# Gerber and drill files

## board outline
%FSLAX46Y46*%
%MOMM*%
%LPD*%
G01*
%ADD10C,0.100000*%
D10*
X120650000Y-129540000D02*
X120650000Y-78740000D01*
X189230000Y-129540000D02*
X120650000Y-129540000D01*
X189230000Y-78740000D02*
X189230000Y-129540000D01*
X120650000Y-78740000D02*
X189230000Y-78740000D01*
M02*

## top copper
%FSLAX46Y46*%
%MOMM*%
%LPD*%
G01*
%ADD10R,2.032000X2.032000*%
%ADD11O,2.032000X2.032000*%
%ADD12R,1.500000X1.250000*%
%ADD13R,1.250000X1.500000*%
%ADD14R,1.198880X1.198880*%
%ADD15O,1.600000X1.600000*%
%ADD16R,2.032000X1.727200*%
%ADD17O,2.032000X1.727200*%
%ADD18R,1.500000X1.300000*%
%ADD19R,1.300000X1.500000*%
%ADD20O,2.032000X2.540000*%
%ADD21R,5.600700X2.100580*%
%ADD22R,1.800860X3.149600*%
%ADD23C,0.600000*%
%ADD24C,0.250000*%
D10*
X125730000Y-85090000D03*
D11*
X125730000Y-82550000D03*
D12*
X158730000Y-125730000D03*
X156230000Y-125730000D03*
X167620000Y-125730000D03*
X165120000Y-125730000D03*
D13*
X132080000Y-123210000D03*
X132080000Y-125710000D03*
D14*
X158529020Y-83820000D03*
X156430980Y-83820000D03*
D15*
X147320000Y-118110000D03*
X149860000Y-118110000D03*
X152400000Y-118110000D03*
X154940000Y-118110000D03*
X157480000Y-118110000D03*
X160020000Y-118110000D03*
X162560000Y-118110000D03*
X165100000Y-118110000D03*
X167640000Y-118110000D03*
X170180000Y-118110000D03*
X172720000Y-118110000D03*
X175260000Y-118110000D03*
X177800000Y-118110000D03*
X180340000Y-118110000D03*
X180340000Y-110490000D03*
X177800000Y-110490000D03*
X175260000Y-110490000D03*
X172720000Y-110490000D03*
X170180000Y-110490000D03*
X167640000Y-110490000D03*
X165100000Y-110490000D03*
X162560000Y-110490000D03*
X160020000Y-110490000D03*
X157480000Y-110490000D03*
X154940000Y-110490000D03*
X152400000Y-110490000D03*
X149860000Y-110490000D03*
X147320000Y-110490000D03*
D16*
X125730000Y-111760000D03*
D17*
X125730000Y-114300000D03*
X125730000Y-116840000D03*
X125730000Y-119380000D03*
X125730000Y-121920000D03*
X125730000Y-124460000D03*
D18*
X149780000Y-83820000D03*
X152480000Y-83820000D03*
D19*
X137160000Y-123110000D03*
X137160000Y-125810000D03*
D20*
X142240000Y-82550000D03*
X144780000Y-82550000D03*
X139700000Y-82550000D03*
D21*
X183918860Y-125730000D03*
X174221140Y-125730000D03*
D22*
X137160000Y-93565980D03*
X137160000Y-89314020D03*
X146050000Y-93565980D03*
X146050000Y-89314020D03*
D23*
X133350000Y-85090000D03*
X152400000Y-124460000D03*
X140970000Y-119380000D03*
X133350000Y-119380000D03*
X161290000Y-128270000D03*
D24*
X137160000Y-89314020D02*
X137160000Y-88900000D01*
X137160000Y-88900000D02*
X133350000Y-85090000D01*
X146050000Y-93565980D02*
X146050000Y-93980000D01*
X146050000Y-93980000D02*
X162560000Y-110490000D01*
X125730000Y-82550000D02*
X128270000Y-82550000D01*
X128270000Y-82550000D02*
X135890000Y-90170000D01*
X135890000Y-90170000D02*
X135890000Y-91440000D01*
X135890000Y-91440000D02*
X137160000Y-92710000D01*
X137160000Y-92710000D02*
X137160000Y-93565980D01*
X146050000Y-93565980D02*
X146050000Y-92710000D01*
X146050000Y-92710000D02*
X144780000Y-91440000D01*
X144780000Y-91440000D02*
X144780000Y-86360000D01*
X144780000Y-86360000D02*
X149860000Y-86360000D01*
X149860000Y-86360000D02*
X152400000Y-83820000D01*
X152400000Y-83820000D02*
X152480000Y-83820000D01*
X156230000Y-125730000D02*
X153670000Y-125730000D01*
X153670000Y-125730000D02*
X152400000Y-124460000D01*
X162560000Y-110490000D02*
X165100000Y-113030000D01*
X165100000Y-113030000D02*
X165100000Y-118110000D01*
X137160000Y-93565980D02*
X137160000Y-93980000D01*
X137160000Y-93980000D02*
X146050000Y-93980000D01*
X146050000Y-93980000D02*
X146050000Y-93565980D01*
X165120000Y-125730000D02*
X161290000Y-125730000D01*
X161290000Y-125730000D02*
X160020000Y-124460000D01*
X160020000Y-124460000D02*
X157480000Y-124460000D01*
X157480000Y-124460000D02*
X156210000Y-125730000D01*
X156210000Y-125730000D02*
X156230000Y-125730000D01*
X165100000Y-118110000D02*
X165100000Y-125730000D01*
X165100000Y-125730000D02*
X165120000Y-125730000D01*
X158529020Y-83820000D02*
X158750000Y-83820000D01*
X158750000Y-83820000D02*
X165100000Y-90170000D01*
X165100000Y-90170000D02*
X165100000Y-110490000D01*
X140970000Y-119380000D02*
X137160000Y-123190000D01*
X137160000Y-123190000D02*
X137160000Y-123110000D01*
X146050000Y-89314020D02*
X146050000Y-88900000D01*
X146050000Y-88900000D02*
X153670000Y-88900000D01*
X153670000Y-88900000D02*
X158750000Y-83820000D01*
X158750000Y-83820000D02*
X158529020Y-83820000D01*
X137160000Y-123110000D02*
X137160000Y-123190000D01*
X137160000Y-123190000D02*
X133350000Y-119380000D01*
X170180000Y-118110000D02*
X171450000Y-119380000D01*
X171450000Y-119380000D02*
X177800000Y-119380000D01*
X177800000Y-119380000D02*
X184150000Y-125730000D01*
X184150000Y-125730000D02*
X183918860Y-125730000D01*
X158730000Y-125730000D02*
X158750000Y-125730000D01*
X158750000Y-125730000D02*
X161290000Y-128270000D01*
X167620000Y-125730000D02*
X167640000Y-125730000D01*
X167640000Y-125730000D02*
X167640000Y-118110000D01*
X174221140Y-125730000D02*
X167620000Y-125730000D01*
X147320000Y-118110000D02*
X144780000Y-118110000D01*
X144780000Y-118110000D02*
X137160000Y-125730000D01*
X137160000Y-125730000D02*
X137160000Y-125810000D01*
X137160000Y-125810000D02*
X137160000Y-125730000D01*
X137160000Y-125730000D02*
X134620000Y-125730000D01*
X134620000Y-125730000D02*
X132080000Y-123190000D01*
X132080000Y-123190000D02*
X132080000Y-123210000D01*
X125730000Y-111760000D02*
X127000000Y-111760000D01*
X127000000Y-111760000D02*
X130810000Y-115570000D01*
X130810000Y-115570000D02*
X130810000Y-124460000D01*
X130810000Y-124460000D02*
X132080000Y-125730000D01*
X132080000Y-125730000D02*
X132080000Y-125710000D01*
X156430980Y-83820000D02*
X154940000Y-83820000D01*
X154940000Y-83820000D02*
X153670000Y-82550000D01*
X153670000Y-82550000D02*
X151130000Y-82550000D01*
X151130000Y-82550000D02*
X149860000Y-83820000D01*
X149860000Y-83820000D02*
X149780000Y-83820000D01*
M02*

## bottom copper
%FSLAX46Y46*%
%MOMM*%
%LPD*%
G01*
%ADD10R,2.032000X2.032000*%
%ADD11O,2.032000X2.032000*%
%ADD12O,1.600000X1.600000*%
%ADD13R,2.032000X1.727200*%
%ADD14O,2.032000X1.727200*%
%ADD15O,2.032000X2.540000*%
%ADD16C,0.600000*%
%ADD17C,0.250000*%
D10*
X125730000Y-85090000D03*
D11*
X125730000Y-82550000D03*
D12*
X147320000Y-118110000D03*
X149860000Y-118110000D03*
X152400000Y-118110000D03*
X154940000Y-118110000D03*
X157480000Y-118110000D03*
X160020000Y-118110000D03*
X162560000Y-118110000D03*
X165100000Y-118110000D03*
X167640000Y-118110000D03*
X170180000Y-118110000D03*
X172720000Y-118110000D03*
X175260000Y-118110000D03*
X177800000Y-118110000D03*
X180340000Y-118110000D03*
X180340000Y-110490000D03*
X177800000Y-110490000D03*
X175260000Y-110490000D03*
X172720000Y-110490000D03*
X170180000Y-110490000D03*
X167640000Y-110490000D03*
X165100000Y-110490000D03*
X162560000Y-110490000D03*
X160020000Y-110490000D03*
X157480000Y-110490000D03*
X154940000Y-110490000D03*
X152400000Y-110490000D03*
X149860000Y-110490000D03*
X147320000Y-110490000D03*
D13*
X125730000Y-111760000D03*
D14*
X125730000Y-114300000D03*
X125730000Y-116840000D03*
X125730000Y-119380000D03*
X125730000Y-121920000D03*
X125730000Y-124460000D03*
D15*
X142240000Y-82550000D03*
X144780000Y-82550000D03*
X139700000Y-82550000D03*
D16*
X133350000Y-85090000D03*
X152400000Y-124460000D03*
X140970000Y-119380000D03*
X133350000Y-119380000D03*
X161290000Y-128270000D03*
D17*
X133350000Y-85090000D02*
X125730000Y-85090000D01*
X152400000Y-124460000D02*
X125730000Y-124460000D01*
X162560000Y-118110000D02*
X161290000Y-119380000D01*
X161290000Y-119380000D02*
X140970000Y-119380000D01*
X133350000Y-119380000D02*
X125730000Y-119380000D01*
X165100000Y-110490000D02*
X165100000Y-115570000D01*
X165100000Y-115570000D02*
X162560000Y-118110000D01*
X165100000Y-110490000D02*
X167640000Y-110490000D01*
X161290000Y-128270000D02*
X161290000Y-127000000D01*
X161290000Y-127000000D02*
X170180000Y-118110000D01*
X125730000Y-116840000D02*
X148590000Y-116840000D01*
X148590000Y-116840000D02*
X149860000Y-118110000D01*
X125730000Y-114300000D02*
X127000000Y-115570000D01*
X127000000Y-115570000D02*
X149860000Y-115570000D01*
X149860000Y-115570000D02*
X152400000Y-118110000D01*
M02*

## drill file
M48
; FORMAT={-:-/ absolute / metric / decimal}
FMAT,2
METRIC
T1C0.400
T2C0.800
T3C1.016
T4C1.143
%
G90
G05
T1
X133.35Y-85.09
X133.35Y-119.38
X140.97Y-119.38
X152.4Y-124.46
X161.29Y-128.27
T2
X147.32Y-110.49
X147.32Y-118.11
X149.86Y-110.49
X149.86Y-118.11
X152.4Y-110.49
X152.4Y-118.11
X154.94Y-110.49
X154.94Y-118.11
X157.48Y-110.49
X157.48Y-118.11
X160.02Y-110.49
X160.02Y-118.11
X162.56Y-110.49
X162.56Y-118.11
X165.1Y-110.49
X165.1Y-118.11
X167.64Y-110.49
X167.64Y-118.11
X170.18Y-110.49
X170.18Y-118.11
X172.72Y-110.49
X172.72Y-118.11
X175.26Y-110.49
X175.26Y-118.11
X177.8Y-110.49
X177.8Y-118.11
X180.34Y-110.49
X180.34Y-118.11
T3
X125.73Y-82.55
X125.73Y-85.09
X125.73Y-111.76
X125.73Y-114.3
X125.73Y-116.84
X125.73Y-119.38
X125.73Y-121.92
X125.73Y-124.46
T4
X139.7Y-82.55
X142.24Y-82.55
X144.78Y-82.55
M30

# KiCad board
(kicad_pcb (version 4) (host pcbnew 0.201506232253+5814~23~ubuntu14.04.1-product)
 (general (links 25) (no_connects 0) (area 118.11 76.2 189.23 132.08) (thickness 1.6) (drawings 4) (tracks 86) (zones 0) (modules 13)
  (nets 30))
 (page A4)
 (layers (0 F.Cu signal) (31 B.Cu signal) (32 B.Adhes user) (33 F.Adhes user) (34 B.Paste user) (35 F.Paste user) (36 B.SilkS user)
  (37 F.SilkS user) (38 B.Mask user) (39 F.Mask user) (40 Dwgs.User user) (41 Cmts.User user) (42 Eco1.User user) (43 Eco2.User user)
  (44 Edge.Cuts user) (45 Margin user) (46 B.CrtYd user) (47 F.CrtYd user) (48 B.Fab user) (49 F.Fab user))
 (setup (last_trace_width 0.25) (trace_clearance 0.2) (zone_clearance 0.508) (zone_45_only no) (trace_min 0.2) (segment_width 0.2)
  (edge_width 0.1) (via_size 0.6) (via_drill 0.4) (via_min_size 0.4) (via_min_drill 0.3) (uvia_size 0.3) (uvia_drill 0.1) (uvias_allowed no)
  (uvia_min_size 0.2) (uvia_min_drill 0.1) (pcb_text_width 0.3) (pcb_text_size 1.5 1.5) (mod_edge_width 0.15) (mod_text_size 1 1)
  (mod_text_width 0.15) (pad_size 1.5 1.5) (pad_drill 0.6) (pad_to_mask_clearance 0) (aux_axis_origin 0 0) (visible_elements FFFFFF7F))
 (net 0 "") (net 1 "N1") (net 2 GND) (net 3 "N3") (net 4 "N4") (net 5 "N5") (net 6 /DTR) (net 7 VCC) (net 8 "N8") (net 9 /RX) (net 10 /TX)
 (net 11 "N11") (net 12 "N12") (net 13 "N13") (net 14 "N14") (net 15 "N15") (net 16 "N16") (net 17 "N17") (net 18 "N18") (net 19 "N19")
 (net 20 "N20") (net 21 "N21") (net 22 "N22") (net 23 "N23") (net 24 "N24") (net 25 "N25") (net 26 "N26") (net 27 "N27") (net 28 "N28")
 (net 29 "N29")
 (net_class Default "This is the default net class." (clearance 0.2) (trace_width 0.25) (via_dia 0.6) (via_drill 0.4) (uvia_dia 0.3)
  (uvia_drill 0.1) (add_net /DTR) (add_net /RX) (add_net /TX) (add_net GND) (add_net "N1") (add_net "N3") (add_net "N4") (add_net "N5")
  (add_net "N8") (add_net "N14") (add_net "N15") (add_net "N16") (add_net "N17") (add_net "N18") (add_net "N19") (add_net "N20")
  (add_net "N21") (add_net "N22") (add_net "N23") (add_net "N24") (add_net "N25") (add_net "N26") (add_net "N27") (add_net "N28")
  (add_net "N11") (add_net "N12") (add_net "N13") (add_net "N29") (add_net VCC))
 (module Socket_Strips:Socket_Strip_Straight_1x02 (layer F.Cu) (at 125.73 85.09 90)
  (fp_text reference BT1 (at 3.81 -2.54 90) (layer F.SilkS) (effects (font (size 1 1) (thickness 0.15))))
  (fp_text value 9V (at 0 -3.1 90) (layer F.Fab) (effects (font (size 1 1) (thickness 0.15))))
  (pad 1 thru_hole rect (at 0 0 90) (size 2.032 2.032) (drill 1.016) (layers *.Cu *.Mask F.SilkS) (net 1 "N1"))
  (pad 2 thru_hole oval (at 2.54 0 90) (size 2.032 2.032) (drill 1.016) (layers *.Cu *.Mask F.SilkS) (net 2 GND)))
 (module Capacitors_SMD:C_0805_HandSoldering (layer F.Cu) (at 157.48 125.73 180)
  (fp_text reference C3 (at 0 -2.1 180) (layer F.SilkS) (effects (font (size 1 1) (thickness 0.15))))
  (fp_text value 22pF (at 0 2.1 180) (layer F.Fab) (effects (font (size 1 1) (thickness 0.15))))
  (pad 1 smd rect (at -1.25 0 180) (size 1.5 1.25) (layers F.Cu F.Paste F.Mask) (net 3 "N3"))
  (pad 2 smd rect (at 1.25 0 180) (size 1.5 1.25) (layers F.Cu F.Paste F.Mask) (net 2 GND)))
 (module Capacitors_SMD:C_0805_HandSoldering (layer F.Cu) (at 166.37 125.73 180)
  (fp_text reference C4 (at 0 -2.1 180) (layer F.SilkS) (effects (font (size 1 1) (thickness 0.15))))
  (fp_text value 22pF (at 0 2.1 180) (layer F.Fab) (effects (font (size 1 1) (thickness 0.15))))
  (pad 1 smd rect (at -1.25 0 180) (size 1.5 1.25) (layers F.Cu F.Paste F.Mask) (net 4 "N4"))
  (pad 2 smd rect (at 1.25 0 180) (size 1.5 1.25) (layers F.Cu F.Paste F.Mask) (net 2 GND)))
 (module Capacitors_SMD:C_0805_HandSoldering (layer F.Cu) (at 132.08 124.46 270)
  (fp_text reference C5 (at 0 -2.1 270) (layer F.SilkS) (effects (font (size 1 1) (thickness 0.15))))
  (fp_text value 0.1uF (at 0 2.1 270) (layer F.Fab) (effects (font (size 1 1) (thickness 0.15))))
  (pad 1 smd rect (at -1.25 0 270) (size 1.5 1.25) (layers F.Cu F.Paste F.Mask) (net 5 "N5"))
  (pad 2 smd rect (at 1.25 0 270) (size 1.5 1.25) (layers F.Cu F.Paste F.Mask) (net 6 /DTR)))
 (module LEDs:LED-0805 (layer F.Cu) (at 157.48 83.82)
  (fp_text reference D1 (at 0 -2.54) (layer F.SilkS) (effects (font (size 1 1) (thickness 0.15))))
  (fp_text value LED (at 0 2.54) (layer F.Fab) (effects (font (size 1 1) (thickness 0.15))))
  (pad 2 smd rect (at 1.04902 0 180) (size 1.19888 1.19888) (layers F.Cu F.Paste F.Mask) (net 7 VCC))
  (pad 1 smd rect (at -1.04902 0 180) (size 1.19888 1.19888) (layers F.Cu F.Paste F.Mask) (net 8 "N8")))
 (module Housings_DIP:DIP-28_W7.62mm (layer F.Cu) (at 147.32 118.11 90)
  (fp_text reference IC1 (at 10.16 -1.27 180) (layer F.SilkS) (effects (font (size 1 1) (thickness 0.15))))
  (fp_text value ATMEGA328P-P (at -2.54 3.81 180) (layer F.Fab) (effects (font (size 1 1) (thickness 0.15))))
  (pad 1 thru_hole oval (at 0 0 90) (size 1.6 1.6) (drill 0.8) (layers *.Cu *.Mask F.SilkS) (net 5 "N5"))
  (pad 2 thru_hole oval (at 0 2.54 90) (size 1.6 1.6) (drill 0.8) (layers *.Cu *.Mask F.SilkS) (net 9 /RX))
  (pad 3 thru_hole oval (at 0 5.08 90) (size 1.6 1.6) (drill 0.8) (layers *.Cu *.Mask F.SilkS) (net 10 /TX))
  (pad 4 thru_hole oval (at 0 7.62 90) (size 1.6 1.6) (drill 0.8) (layers *.Cu *.Mask F.SilkS) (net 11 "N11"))
  (pad 5 thru_hole oval (at 0 10.16 90) (size 1.6 1.6) (drill 0.8) (layers *.Cu *.Mask F.SilkS) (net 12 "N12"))
  (pad 6 thru_hole oval (at 0 12.7 90) (size 1.6 1.6) (drill 0.8) (layers *.Cu *.Mask F.SilkS) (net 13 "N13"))
  (pad 7 thru_hole oval (at 0 15.24 90) (size 1.6 1.6) (drill 0.8) (layers *.Cu *.Mask F.SilkS) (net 7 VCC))
  (pad 8 thru_hole oval (at 0 17.78 90) (size 1.6 1.6) (drill 0.8) (layers *.Cu *.Mask F.SilkS) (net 2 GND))
  (pad 9 thru_hole oval (at 0 20.32 90) (size 1.6 1.6) (drill 0.8) (layers *.Cu *.Mask F.SilkS) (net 4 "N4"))
  (pad 10 thru_hole oval (at 0 22.86 90) (size 1.6 1.6) (drill 0.8) (layers *.Cu *.Mask F.SilkS) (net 3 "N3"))
  (pad 11 thru_hole oval (at 0 25.4 90) (size 1.6 1.6) (drill 0.8) (layers *.Cu *.Mask F.SilkS) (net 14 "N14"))
  (pad 12 thru_hole oval (at 0 27.94 90) (size 1.6 1.6) (drill 0.8) (layers *.Cu *.Mask F.SilkS) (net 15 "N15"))
  (pad 13 thru_hole oval (at 0 30.48 90) (size 1.6 1.6) (drill 0.8) (layers *.Cu *.Mask F.SilkS) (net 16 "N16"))
  (pad 14 thru_hole oval (at 0 33.02 90) (size 1.6 1.6) (drill 0.8) (layers *.Cu *.Mask F.SilkS) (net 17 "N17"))
  (pad 15 thru_hole oval (at 7.62 33.02 90) (size 1.6 1.6) (drill 0.8) (layers *.Cu *.Mask F.SilkS) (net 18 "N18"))
  (pad 16 thru_hole oval (at 7.62 30.48 90) (size 1.6 1.6) (drill 0.8) (layers *.Cu *.Mask F.SilkS) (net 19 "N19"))
  (pad 17 thru_hole oval (at 7.62 27.94 90) (size 1.6 1.6) (drill 0.8) (layers *.Cu *.Mask F.SilkS) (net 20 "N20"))
  (pad 18 thru_hole oval (at 7.62 25.4 90) (size 1.6 1.6) (drill 0.8) (layers *.Cu *.Mask F.SilkS) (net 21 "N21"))
  (pad 19 thru_hole oval (at 7.62 22.86 90) (size 1.6 1.6) (drill 0.8) (layers *.Cu *.Mask F.SilkS) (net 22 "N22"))
  (pad 20 thru_hole oval (at 7.62 20.32 90) (size 1.6 1.6) (drill 0.8) (layers *.Cu *.Mask F.SilkS) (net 7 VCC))
  (pad 21 thru_hole oval (at 7.62 17.78 90) (size 1.6 1.6) (drill 0.8) (layers *.Cu *.Mask F.SilkS) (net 7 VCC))
  (pad 22 thru_hole oval (at 7.62 15.24 90) (size 1.6 1.6) (drill 0.8) (layers *.Cu *.Mask F.SilkS) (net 2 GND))
  (pad 23 thru_hole oval (at 7.62 12.7 90) (size 1.6 1.6) (drill 0.8) (layers *.Cu *.Mask F.SilkS) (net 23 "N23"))
  (pad 24 thru_hole oval (at 7.62 10.16 90) (size 1.6 1.6) (drill 0.8) (layers *.Cu *.Mask F.SilkS) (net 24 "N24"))
  (pad 25 thru_hole oval (at 7.62 7.62 90) (size 1.6 1.6) (drill 0.8) (layers *.Cu *.Mask F.SilkS) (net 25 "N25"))
  (pad 26 thru_hole oval (at 7.62 5.08 90) (size 1.6 1.6) (drill 0.8) (layers *.Cu *.Mask F.SilkS) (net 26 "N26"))
  (pad 27 thru_hole oval (at 7.62 2.54 90) (size 1.6 1.6) (drill 0.8) (layers *.Cu *.Mask F.SilkS) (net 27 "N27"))
  (pad 28 thru_hole oval (at 7.62 0 90) (size 1.6 1.6) (drill 0.8) (layers *.Cu *.Mask F.SilkS) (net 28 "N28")))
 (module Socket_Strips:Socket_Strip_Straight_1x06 (layer F.Cu) (at 125.73 111.76 270)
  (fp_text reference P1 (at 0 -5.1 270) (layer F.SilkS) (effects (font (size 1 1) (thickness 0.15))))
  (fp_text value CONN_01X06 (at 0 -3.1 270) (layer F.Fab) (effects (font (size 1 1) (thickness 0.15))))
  (pad 1 thru_hole rect (at 0 0 270) (size 1.7272 2.032) (drill 1.016) (layers *.Cu *.Mask F.SilkS) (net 6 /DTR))
  (pad 2 thru_hole oval (at 2.54 0 270) (size 1.7272 2.032) (drill 1.016) (layers *.Cu *.Mask F.SilkS) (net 10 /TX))
  (pad 3 thru_hole oval (at 5.08 0 270) (size 1.7272 2.032) (drill 1.016) (layers *.Cu *.Mask F.SilkS) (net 9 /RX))
  (pad 4 thru_hole oval (at 7.62 0 270) (size 1.7272 2.032) (drill 1.016) (layers *.Cu *.Mask F.SilkS) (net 7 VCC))
  (pad 5 thru_hole oval (at 10.16 0 270) (size 1.7272 2.032) (drill 1.016) (layers *.Cu *.Mask F.SilkS) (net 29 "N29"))
  (pad 6 thru_hole oval (at 12.7 0 270) (size 1.7272 2.032) (drill 1.016) (layers *.Cu *.Mask F.SilkS) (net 2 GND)))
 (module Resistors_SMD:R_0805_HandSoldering (layer F.Cu) (at 151.13 83.82)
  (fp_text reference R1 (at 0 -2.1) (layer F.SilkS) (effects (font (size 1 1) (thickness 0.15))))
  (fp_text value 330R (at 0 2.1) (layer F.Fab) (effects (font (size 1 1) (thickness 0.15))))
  (pad 1 smd rect (at -1.35 0) (size 1.5 1.3) (layers F.Cu F.Paste F.Mask) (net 8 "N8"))
  (pad 2 smd rect (at 1.35 0) (size 1.5 1.3) (layers F.Cu F.Paste F.Mask) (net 2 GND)))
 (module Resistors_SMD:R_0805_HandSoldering (layer F.Cu) (at 137.16 124.46 270)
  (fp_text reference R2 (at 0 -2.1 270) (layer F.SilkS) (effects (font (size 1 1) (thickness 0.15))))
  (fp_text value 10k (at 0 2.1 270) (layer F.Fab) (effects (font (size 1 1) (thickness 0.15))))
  (pad 1 smd rect (at -1.35 0 270) (size 1.5 1.3) (layers F.Cu F.Paste F.Mask) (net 7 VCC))
  (pad 2 smd rect (at 1.35 0 270) (size 1.5 1.3) (layers F.Cu F.Paste F.Mask) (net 5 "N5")))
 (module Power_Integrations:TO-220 (layer F.Cu) (at 142.24 82.55)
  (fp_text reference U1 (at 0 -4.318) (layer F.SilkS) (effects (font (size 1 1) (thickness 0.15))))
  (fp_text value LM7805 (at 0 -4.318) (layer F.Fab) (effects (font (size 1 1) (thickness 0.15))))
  (pad 2 thru_hole oval (at 0 0) (size 2.032 2.54) (drill 1.143) (layers *.Cu *.Mask F.SilkS))
  (pad 3 thru_hole oval (at 2.54 0) (size 2.032 2.54) (drill 1.143) (layers *.Cu *.Mask F.SilkS))
  (pad 1 thru_hole oval (at -2.54 0) (size 2.032 2.54) (drill 1.143) (layers *.Cu *.Mask F.SilkS)))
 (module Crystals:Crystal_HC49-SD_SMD (layer F.Cu) (at 179.07 125.73 180)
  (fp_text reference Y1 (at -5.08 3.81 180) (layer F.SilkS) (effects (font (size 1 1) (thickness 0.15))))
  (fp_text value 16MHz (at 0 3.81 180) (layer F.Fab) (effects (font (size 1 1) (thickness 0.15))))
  (pad 1 smd rect (at -4.84886 0 180) (size 5.6007 2.10058) (layers F.Cu F.Paste F.Mask) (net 3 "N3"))
  (pad 2 smd rect (at 4.84886 0 180) (size 5.6007 2.10058) (layers F.Cu F.Paste F.Mask) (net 4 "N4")))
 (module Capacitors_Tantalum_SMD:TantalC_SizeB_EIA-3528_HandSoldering (layer F.Cu) (at 137.16 91.44 270)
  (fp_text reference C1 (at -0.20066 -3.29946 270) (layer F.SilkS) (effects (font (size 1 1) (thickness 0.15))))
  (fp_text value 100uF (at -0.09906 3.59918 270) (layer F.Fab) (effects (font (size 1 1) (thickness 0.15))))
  (pad 2 smd rect (at 2.12598 0 270) (size 3.1496 1.80086) (layers F.Cu F.Paste F.Mask) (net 2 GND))
  (pad 1 smd rect (at -2.12598 0 270) (size 3.1496 1.80086) (layers F.Cu F.Paste F.Mask) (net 1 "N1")))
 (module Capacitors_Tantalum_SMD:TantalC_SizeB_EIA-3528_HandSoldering (layer F.Cu) (at 146.05 91.44 270)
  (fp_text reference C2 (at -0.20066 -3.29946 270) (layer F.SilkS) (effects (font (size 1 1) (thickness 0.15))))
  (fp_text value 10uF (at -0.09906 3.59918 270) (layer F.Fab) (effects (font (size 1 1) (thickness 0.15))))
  (pad 2 smd rect (at 2.12598 0 270) (size 3.1496 1.80086) (layers F.Cu F.Paste F.Mask) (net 2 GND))
  (pad 1 smd rect (at -2.12598 0 270) (size 3.1496 1.80086) (layers F.Cu F.Paste F.Mask) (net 7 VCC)))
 (gr_line (start 120.65 129.54) (end 120.65 78.74) (angle 90) (layer Edge.Cuts) (width 0.1))
 (gr_line (start 189.23 129.54) (end 120.65 129.54) (angle 90) (layer Edge.Cuts) (width 0.1))
 (gr_line (start 189.23 78.74) (end 189.23 129.54) (angle 90) (layer Edge.Cuts) (width 0.1))
 (gr_line (start 120.65 78.74) (end 189.23 78.74) (angle 90) (layer Edge.Cuts) (width 0.1))
 (segment (start 137.16 89.31402) (end 137.16 88.9) (width 0.25) (layer F.Cu) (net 1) (status 80000))
 (segment (start 137.16 88.9) (end 133.35 85.09) (width 0.25) (layer F.Cu) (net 1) (status 80000))
 (via (at 133.35 85.09) (size 0.6) (layers F.Cu B.Cu) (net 1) (status 80000))
 (segment (start 133.35 85.09) (end 125.73 85.09) (width 0.25) (layer B.Cu) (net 1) (status 80000))
 (segment (start 146.05 93.56598) (end 146.05 93.98) (width 0.25) (layer F.Cu) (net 2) (status 80000))
 (segment (start 146.05 93.98) (end 162.56 110.49) (width 0.25) (layer F.Cu) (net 2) (status 80000))
 (segment (start 125.73 82.55) (end 128.27 82.55) (width 0.25) (layer F.Cu) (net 2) (status 80000))
 (segment (start 128.27 82.55) (end 135.89 90.17) (width 0.25) (layer F.Cu) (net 2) (status 80000))
 (segment (start 135.89 90.17) (end 135.89 91.44) (width 0.25) (layer F.Cu) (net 2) (status 80000))
 (segment (start 135.89 91.44) (end 137.16 92.71) (width 0.25) (layer F.Cu) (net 2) (status 80000))
 (segment (start 137.16 92.71) (end 137.16 93.56598) (width 0.25) (layer F.Cu) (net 2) (status 80000))
 (segment (start 146.05 93.56598) (end 146.05 92.71) (width 0.25) (layer F.Cu) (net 2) (status 80000))
 (segment (start 146.05 92.71) (end 144.78 91.44) (width 0.25) (layer F.Cu) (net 2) (status 80000))
 (segment (start 144.78 91.44) (end 144.78 86.36) (width 0.25) (layer F.Cu) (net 2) (status 80000))
 (segment (start 144.78 86.36) (end 149.86 86.36) (width 0.25) (layer F.Cu) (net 2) (status 80000))
 (segment (start 149.86 86.36) (end 152.4 83.82) (width 0.25) (layer F.Cu) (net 2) (status 80000))
 (segment (start 152.4 83.82) (end 152.48 83.82) (width 0.25) (layer F.Cu) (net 2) (status 80000))
 (segment (start 156.23 125.73) (end 153.67 125.73) (width 0.25) (layer F.Cu) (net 2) (status 80000))
 (segment (start 153.67 125.73) (end 152.4 124.46) (width 0.25) (layer F.Cu) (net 2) (status 80000))
 (via (at 152.4 124.46) (size 0.6) (layers F.Cu B.Cu) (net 2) (status 80000))
 (segment (start 152.4 124.46) (end 125.73 124.46) (width 0.25) (layer B.Cu) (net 2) (status 80000))
 (segment (start 162.56 110.49) (end 165.1 113.03) (width 0.25) (layer F.Cu) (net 2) (status 80000))
 (segment (start 165.1 113.03) (end 165.1 118.11) (width 0.25) (layer F.Cu) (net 2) (status 80000))
 (segment (start 137.16 93.56598) (end 137.16 93.98) (width 0.25) (layer F.Cu) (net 2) (status 80000))
 (segment (start 137.16 93.98) (end 146.05 93.98) (width 0.25) (layer F.Cu) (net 2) (status 80000))
 (segment (start 146.05 93.98) (end 146.05 93.56598) (width 0.25) (layer F.Cu) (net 2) (status 80000))
 (segment (start 165.12 125.73) (end 161.29 125.73) (width 0.25) (layer F.Cu) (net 2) (status 80000))
 (segment (start 161.29 125.73) (end 160.02 124.46) (width 0.25) (layer F.Cu) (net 2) (status 80000))
 (segment (start 160.02 124.46) (end 157.48 124.46) (width 0.25) (layer F.Cu) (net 2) (status 80000))
 (segment (start 157.48 124.46) (end 156.21 125.73) (width 0.25) (layer F.Cu) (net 2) (status 80000))
 (segment (start 156.21 125.73) (end 156.23 125.73) (width 0.25) (layer F.Cu) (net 2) (status 80000))
 (segment (start 165.1 118.11) (end 165.1 125.73) (width 0.25) (layer F.Cu) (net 2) (status 80000))
 (segment (start 165.1 125.73) (end 165.12 125.73) (width 0.25) (layer F.Cu) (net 2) (status 80000))
 (segment (start 158.52902 83.82) (end 158.75 83.82) (width 0.25) (layer F.Cu) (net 7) (status 80000))
 (segment (start 158.75 83.82) (end 165.1 90.17) (width 0.25) (layer F.Cu) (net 7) (status 80000))
 (segment (start 165.1 90.17) (end 165.1 110.49) (width 0.25) (layer F.Cu) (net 7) (status 80000))
 (segment (start 162.56 118.11) (end 161.29 119.38) (width 0.25) (layer B.Cu) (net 7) (status 80000))
 (segment (start 161.29 119.38) (end 140.97 119.38) (width 0.25) (layer B.Cu) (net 7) (status 80000))
 (via (at 140.97 119.38) (size 0.6) (layers F.Cu B.Cu) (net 7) (status 80000))
 (segment (start 140.97 119.38) (end 137.16 123.19) (width 0.25) (layer F.Cu) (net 7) (status 80000))
 (segment (start 137.16 123.19) (end 137.16 123.11) (width 0.25) (layer F.Cu) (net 7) (status 80000))
 (segment (start 146.05 89.31402) (end 146.05 88.9) (width 0.25) (layer F.Cu) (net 7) (status 80000))
 (segment (start 146.05 88.9) (end 153.67 88.9) (width 0.25) (layer F.Cu) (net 7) (status 80000))
 (segment (start 153.67 88.9) (end 158.75 83.82) (width 0.25) (layer F.Cu) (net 7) (status 80000))
 (segment (start 158.75 83.82) (end 158.52902 83.82) (width 0.25) (layer F.Cu) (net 7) (status 80000))
 (segment (start 137.16 123.11) (end 137.16 123.19) (width 0.25) (layer F.Cu) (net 7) (status 80000))
 (segment (start 137.16 123.19) (end 133.35 119.38) (width 0.25) (layer F.Cu) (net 7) (status 80000))
 (via (at 133.35 119.38) (size 0.6) (layers F.Cu B.Cu) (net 7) (status 80000))
 (segment (start 133.35 119.38) (end 125.73 119.38) (width 0.25) (layer B.Cu) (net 7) (status 80000))
 (segment (start 165.1 110.49) (end 165.1 115.57) (width 0.25) (layer B.Cu) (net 7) (status 80000))
 (segment (start 165.1 115.57) (end 162.56 118.11) (width 0.25) (layer B.Cu) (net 7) (status 80000))
 (segment (start 165.1 110.49) (end 167.64 110.49) (width 0.25) (layer B.Cu) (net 7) (status 80000))
 (segment (start 170.18 118.11) (end 171.45 119.38) (width 0.25) (layer F.Cu) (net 3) (status 80000))
 (segment (start 171.45 119.38) (end 177.8 119.38) (width 0.25) (layer F.Cu) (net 3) (status 80000))
 (segment (start 177.8 119.38) (end 184.15 125.73) (width 0.25) (layer F.Cu) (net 3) (status 80000))
 (segment (start 184.15 125.73) (end 183.91886 125.73) (width 0.25) (layer F.Cu) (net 3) (status 80000))
 (segment (start 158.73 125.73) (end 158.75 125.73) (width 0.25) (layer F.Cu) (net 3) (status 80000))
 (segment (start 158.75 125.73) (end 161.29 128.27) (width 0.25) (layer F.Cu) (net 3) (status 80000))
 (via (at 161.29 128.27) (size 0.6) (layers F.Cu B.Cu) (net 3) (status 80000))
 (segment (start 161.29 128.27) (end 161.29 127) (width 0.25) (layer B.Cu) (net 3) (status 80000))
 (segment (start 161.29 127) (end 170.18 118.11) (width 0.25) (layer B.Cu) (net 3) (status 80000))
 (segment (start 167.62 125.73) (end 167.64 125.73) (width 0.25) (layer F.Cu) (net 4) (status 80000))
 (segment (start 167.64 125.73) (end 167.64 118.11) (width 0.25) (layer F.Cu) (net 4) (status 80000))
 (segment (start 174.22114 125.73) (end 167.62 125.73) (width 0.25) (layer F.Cu) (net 4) (status 80000))
 (segment (start 147.32 118.11) (end 144.78 118.11) (width 0.25) (layer F.Cu) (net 5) (status 80000))
 (segment (start 144.78 118.11) (end 137.16 125.73) (width 0.25) (layer F.Cu) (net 5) (status 80000))
 (segment (start 137.16 125.73) (end 137.16 125.81) (width 0.25) (layer F.Cu) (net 5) (status 80000))
 (segment (start 137.16 125.81) (end 137.16 125.73) (width 0.25) (layer F.Cu) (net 5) (status 80000))
 (segment (start 137.16 125.73) (end 134.62 125.73) (width 0.25) (layer F.Cu) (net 5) (status 80000))
 (segment (start 134.62 125.73) (end 132.08 123.19) (width 0.25) (layer F.Cu) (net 5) (status 80000))
 (segment (start 132.08 123.19) (end 132.08 123.21) (width 0.25) (layer F.Cu) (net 5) (status 80000))
 (segment (start 125.73 111.76) (end 127 111.76) (width 0.25) (layer F.Cu) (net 6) (status 80000))
 (segment (start 127 111.76) (end 130.81 115.57) (width 0.25) (layer F.Cu) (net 6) (status 80000))
 (segment (start 130.81 115.57) (end 130.81 124.46) (width 0.25) (layer F.Cu) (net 6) (status 80000))
 (segment (start 130.81 124.46) (end 132.08 125.73) (width 0.25) (layer F.Cu) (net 6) (status 80000))
 (segment (start 132.08 125.73) (end 132.08 125.71) (width 0.25) (layer F.Cu) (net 6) (status 80000))
 (segment (start 156.43098 83.82) (end 154.94 83.82) (width 0.25) (layer F.Cu) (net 8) (status 80000))
 (segment (start 154.94 83.82) (end 153.67 82.55) (width 0.25) (layer F.Cu) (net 8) (status 80000))
 (segment (start 153.67 82.55) (end 151.13 82.55) (width 0.25) (layer F.Cu) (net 8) (status 80000))
 (segment (start 151.13 82.55) (end 149.86 83.82) (width 0.25) (layer F.Cu) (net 8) (status 80000))
 (segment (start 149.86 83.82) (end 149.78 83.82) (width 0.25) (layer F.Cu) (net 8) (status 80000))
 (segment (start 125.73 116.84) (end 148.59 116.84) (width 0.25) (layer B.Cu) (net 9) (status 80000))
 (segment (start 148.59 116.84) (end 149.86 118.11) (width 0.25) (layer B.Cu) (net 9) (status 80000))
 (segment (start 125.73 114.3) (end 127 115.57) (width 0.25) (layer B.Cu) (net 10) (status 80000))
 (segment (start 127 115.57) (end 149.86 115.57) (width 0.25) (layer B.Cu) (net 10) (status 80000))
 (segment (start 149.86 115.57) (end 152.4 118.11) (width 0.25) (layer B.Cu) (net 10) (status 80000)))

